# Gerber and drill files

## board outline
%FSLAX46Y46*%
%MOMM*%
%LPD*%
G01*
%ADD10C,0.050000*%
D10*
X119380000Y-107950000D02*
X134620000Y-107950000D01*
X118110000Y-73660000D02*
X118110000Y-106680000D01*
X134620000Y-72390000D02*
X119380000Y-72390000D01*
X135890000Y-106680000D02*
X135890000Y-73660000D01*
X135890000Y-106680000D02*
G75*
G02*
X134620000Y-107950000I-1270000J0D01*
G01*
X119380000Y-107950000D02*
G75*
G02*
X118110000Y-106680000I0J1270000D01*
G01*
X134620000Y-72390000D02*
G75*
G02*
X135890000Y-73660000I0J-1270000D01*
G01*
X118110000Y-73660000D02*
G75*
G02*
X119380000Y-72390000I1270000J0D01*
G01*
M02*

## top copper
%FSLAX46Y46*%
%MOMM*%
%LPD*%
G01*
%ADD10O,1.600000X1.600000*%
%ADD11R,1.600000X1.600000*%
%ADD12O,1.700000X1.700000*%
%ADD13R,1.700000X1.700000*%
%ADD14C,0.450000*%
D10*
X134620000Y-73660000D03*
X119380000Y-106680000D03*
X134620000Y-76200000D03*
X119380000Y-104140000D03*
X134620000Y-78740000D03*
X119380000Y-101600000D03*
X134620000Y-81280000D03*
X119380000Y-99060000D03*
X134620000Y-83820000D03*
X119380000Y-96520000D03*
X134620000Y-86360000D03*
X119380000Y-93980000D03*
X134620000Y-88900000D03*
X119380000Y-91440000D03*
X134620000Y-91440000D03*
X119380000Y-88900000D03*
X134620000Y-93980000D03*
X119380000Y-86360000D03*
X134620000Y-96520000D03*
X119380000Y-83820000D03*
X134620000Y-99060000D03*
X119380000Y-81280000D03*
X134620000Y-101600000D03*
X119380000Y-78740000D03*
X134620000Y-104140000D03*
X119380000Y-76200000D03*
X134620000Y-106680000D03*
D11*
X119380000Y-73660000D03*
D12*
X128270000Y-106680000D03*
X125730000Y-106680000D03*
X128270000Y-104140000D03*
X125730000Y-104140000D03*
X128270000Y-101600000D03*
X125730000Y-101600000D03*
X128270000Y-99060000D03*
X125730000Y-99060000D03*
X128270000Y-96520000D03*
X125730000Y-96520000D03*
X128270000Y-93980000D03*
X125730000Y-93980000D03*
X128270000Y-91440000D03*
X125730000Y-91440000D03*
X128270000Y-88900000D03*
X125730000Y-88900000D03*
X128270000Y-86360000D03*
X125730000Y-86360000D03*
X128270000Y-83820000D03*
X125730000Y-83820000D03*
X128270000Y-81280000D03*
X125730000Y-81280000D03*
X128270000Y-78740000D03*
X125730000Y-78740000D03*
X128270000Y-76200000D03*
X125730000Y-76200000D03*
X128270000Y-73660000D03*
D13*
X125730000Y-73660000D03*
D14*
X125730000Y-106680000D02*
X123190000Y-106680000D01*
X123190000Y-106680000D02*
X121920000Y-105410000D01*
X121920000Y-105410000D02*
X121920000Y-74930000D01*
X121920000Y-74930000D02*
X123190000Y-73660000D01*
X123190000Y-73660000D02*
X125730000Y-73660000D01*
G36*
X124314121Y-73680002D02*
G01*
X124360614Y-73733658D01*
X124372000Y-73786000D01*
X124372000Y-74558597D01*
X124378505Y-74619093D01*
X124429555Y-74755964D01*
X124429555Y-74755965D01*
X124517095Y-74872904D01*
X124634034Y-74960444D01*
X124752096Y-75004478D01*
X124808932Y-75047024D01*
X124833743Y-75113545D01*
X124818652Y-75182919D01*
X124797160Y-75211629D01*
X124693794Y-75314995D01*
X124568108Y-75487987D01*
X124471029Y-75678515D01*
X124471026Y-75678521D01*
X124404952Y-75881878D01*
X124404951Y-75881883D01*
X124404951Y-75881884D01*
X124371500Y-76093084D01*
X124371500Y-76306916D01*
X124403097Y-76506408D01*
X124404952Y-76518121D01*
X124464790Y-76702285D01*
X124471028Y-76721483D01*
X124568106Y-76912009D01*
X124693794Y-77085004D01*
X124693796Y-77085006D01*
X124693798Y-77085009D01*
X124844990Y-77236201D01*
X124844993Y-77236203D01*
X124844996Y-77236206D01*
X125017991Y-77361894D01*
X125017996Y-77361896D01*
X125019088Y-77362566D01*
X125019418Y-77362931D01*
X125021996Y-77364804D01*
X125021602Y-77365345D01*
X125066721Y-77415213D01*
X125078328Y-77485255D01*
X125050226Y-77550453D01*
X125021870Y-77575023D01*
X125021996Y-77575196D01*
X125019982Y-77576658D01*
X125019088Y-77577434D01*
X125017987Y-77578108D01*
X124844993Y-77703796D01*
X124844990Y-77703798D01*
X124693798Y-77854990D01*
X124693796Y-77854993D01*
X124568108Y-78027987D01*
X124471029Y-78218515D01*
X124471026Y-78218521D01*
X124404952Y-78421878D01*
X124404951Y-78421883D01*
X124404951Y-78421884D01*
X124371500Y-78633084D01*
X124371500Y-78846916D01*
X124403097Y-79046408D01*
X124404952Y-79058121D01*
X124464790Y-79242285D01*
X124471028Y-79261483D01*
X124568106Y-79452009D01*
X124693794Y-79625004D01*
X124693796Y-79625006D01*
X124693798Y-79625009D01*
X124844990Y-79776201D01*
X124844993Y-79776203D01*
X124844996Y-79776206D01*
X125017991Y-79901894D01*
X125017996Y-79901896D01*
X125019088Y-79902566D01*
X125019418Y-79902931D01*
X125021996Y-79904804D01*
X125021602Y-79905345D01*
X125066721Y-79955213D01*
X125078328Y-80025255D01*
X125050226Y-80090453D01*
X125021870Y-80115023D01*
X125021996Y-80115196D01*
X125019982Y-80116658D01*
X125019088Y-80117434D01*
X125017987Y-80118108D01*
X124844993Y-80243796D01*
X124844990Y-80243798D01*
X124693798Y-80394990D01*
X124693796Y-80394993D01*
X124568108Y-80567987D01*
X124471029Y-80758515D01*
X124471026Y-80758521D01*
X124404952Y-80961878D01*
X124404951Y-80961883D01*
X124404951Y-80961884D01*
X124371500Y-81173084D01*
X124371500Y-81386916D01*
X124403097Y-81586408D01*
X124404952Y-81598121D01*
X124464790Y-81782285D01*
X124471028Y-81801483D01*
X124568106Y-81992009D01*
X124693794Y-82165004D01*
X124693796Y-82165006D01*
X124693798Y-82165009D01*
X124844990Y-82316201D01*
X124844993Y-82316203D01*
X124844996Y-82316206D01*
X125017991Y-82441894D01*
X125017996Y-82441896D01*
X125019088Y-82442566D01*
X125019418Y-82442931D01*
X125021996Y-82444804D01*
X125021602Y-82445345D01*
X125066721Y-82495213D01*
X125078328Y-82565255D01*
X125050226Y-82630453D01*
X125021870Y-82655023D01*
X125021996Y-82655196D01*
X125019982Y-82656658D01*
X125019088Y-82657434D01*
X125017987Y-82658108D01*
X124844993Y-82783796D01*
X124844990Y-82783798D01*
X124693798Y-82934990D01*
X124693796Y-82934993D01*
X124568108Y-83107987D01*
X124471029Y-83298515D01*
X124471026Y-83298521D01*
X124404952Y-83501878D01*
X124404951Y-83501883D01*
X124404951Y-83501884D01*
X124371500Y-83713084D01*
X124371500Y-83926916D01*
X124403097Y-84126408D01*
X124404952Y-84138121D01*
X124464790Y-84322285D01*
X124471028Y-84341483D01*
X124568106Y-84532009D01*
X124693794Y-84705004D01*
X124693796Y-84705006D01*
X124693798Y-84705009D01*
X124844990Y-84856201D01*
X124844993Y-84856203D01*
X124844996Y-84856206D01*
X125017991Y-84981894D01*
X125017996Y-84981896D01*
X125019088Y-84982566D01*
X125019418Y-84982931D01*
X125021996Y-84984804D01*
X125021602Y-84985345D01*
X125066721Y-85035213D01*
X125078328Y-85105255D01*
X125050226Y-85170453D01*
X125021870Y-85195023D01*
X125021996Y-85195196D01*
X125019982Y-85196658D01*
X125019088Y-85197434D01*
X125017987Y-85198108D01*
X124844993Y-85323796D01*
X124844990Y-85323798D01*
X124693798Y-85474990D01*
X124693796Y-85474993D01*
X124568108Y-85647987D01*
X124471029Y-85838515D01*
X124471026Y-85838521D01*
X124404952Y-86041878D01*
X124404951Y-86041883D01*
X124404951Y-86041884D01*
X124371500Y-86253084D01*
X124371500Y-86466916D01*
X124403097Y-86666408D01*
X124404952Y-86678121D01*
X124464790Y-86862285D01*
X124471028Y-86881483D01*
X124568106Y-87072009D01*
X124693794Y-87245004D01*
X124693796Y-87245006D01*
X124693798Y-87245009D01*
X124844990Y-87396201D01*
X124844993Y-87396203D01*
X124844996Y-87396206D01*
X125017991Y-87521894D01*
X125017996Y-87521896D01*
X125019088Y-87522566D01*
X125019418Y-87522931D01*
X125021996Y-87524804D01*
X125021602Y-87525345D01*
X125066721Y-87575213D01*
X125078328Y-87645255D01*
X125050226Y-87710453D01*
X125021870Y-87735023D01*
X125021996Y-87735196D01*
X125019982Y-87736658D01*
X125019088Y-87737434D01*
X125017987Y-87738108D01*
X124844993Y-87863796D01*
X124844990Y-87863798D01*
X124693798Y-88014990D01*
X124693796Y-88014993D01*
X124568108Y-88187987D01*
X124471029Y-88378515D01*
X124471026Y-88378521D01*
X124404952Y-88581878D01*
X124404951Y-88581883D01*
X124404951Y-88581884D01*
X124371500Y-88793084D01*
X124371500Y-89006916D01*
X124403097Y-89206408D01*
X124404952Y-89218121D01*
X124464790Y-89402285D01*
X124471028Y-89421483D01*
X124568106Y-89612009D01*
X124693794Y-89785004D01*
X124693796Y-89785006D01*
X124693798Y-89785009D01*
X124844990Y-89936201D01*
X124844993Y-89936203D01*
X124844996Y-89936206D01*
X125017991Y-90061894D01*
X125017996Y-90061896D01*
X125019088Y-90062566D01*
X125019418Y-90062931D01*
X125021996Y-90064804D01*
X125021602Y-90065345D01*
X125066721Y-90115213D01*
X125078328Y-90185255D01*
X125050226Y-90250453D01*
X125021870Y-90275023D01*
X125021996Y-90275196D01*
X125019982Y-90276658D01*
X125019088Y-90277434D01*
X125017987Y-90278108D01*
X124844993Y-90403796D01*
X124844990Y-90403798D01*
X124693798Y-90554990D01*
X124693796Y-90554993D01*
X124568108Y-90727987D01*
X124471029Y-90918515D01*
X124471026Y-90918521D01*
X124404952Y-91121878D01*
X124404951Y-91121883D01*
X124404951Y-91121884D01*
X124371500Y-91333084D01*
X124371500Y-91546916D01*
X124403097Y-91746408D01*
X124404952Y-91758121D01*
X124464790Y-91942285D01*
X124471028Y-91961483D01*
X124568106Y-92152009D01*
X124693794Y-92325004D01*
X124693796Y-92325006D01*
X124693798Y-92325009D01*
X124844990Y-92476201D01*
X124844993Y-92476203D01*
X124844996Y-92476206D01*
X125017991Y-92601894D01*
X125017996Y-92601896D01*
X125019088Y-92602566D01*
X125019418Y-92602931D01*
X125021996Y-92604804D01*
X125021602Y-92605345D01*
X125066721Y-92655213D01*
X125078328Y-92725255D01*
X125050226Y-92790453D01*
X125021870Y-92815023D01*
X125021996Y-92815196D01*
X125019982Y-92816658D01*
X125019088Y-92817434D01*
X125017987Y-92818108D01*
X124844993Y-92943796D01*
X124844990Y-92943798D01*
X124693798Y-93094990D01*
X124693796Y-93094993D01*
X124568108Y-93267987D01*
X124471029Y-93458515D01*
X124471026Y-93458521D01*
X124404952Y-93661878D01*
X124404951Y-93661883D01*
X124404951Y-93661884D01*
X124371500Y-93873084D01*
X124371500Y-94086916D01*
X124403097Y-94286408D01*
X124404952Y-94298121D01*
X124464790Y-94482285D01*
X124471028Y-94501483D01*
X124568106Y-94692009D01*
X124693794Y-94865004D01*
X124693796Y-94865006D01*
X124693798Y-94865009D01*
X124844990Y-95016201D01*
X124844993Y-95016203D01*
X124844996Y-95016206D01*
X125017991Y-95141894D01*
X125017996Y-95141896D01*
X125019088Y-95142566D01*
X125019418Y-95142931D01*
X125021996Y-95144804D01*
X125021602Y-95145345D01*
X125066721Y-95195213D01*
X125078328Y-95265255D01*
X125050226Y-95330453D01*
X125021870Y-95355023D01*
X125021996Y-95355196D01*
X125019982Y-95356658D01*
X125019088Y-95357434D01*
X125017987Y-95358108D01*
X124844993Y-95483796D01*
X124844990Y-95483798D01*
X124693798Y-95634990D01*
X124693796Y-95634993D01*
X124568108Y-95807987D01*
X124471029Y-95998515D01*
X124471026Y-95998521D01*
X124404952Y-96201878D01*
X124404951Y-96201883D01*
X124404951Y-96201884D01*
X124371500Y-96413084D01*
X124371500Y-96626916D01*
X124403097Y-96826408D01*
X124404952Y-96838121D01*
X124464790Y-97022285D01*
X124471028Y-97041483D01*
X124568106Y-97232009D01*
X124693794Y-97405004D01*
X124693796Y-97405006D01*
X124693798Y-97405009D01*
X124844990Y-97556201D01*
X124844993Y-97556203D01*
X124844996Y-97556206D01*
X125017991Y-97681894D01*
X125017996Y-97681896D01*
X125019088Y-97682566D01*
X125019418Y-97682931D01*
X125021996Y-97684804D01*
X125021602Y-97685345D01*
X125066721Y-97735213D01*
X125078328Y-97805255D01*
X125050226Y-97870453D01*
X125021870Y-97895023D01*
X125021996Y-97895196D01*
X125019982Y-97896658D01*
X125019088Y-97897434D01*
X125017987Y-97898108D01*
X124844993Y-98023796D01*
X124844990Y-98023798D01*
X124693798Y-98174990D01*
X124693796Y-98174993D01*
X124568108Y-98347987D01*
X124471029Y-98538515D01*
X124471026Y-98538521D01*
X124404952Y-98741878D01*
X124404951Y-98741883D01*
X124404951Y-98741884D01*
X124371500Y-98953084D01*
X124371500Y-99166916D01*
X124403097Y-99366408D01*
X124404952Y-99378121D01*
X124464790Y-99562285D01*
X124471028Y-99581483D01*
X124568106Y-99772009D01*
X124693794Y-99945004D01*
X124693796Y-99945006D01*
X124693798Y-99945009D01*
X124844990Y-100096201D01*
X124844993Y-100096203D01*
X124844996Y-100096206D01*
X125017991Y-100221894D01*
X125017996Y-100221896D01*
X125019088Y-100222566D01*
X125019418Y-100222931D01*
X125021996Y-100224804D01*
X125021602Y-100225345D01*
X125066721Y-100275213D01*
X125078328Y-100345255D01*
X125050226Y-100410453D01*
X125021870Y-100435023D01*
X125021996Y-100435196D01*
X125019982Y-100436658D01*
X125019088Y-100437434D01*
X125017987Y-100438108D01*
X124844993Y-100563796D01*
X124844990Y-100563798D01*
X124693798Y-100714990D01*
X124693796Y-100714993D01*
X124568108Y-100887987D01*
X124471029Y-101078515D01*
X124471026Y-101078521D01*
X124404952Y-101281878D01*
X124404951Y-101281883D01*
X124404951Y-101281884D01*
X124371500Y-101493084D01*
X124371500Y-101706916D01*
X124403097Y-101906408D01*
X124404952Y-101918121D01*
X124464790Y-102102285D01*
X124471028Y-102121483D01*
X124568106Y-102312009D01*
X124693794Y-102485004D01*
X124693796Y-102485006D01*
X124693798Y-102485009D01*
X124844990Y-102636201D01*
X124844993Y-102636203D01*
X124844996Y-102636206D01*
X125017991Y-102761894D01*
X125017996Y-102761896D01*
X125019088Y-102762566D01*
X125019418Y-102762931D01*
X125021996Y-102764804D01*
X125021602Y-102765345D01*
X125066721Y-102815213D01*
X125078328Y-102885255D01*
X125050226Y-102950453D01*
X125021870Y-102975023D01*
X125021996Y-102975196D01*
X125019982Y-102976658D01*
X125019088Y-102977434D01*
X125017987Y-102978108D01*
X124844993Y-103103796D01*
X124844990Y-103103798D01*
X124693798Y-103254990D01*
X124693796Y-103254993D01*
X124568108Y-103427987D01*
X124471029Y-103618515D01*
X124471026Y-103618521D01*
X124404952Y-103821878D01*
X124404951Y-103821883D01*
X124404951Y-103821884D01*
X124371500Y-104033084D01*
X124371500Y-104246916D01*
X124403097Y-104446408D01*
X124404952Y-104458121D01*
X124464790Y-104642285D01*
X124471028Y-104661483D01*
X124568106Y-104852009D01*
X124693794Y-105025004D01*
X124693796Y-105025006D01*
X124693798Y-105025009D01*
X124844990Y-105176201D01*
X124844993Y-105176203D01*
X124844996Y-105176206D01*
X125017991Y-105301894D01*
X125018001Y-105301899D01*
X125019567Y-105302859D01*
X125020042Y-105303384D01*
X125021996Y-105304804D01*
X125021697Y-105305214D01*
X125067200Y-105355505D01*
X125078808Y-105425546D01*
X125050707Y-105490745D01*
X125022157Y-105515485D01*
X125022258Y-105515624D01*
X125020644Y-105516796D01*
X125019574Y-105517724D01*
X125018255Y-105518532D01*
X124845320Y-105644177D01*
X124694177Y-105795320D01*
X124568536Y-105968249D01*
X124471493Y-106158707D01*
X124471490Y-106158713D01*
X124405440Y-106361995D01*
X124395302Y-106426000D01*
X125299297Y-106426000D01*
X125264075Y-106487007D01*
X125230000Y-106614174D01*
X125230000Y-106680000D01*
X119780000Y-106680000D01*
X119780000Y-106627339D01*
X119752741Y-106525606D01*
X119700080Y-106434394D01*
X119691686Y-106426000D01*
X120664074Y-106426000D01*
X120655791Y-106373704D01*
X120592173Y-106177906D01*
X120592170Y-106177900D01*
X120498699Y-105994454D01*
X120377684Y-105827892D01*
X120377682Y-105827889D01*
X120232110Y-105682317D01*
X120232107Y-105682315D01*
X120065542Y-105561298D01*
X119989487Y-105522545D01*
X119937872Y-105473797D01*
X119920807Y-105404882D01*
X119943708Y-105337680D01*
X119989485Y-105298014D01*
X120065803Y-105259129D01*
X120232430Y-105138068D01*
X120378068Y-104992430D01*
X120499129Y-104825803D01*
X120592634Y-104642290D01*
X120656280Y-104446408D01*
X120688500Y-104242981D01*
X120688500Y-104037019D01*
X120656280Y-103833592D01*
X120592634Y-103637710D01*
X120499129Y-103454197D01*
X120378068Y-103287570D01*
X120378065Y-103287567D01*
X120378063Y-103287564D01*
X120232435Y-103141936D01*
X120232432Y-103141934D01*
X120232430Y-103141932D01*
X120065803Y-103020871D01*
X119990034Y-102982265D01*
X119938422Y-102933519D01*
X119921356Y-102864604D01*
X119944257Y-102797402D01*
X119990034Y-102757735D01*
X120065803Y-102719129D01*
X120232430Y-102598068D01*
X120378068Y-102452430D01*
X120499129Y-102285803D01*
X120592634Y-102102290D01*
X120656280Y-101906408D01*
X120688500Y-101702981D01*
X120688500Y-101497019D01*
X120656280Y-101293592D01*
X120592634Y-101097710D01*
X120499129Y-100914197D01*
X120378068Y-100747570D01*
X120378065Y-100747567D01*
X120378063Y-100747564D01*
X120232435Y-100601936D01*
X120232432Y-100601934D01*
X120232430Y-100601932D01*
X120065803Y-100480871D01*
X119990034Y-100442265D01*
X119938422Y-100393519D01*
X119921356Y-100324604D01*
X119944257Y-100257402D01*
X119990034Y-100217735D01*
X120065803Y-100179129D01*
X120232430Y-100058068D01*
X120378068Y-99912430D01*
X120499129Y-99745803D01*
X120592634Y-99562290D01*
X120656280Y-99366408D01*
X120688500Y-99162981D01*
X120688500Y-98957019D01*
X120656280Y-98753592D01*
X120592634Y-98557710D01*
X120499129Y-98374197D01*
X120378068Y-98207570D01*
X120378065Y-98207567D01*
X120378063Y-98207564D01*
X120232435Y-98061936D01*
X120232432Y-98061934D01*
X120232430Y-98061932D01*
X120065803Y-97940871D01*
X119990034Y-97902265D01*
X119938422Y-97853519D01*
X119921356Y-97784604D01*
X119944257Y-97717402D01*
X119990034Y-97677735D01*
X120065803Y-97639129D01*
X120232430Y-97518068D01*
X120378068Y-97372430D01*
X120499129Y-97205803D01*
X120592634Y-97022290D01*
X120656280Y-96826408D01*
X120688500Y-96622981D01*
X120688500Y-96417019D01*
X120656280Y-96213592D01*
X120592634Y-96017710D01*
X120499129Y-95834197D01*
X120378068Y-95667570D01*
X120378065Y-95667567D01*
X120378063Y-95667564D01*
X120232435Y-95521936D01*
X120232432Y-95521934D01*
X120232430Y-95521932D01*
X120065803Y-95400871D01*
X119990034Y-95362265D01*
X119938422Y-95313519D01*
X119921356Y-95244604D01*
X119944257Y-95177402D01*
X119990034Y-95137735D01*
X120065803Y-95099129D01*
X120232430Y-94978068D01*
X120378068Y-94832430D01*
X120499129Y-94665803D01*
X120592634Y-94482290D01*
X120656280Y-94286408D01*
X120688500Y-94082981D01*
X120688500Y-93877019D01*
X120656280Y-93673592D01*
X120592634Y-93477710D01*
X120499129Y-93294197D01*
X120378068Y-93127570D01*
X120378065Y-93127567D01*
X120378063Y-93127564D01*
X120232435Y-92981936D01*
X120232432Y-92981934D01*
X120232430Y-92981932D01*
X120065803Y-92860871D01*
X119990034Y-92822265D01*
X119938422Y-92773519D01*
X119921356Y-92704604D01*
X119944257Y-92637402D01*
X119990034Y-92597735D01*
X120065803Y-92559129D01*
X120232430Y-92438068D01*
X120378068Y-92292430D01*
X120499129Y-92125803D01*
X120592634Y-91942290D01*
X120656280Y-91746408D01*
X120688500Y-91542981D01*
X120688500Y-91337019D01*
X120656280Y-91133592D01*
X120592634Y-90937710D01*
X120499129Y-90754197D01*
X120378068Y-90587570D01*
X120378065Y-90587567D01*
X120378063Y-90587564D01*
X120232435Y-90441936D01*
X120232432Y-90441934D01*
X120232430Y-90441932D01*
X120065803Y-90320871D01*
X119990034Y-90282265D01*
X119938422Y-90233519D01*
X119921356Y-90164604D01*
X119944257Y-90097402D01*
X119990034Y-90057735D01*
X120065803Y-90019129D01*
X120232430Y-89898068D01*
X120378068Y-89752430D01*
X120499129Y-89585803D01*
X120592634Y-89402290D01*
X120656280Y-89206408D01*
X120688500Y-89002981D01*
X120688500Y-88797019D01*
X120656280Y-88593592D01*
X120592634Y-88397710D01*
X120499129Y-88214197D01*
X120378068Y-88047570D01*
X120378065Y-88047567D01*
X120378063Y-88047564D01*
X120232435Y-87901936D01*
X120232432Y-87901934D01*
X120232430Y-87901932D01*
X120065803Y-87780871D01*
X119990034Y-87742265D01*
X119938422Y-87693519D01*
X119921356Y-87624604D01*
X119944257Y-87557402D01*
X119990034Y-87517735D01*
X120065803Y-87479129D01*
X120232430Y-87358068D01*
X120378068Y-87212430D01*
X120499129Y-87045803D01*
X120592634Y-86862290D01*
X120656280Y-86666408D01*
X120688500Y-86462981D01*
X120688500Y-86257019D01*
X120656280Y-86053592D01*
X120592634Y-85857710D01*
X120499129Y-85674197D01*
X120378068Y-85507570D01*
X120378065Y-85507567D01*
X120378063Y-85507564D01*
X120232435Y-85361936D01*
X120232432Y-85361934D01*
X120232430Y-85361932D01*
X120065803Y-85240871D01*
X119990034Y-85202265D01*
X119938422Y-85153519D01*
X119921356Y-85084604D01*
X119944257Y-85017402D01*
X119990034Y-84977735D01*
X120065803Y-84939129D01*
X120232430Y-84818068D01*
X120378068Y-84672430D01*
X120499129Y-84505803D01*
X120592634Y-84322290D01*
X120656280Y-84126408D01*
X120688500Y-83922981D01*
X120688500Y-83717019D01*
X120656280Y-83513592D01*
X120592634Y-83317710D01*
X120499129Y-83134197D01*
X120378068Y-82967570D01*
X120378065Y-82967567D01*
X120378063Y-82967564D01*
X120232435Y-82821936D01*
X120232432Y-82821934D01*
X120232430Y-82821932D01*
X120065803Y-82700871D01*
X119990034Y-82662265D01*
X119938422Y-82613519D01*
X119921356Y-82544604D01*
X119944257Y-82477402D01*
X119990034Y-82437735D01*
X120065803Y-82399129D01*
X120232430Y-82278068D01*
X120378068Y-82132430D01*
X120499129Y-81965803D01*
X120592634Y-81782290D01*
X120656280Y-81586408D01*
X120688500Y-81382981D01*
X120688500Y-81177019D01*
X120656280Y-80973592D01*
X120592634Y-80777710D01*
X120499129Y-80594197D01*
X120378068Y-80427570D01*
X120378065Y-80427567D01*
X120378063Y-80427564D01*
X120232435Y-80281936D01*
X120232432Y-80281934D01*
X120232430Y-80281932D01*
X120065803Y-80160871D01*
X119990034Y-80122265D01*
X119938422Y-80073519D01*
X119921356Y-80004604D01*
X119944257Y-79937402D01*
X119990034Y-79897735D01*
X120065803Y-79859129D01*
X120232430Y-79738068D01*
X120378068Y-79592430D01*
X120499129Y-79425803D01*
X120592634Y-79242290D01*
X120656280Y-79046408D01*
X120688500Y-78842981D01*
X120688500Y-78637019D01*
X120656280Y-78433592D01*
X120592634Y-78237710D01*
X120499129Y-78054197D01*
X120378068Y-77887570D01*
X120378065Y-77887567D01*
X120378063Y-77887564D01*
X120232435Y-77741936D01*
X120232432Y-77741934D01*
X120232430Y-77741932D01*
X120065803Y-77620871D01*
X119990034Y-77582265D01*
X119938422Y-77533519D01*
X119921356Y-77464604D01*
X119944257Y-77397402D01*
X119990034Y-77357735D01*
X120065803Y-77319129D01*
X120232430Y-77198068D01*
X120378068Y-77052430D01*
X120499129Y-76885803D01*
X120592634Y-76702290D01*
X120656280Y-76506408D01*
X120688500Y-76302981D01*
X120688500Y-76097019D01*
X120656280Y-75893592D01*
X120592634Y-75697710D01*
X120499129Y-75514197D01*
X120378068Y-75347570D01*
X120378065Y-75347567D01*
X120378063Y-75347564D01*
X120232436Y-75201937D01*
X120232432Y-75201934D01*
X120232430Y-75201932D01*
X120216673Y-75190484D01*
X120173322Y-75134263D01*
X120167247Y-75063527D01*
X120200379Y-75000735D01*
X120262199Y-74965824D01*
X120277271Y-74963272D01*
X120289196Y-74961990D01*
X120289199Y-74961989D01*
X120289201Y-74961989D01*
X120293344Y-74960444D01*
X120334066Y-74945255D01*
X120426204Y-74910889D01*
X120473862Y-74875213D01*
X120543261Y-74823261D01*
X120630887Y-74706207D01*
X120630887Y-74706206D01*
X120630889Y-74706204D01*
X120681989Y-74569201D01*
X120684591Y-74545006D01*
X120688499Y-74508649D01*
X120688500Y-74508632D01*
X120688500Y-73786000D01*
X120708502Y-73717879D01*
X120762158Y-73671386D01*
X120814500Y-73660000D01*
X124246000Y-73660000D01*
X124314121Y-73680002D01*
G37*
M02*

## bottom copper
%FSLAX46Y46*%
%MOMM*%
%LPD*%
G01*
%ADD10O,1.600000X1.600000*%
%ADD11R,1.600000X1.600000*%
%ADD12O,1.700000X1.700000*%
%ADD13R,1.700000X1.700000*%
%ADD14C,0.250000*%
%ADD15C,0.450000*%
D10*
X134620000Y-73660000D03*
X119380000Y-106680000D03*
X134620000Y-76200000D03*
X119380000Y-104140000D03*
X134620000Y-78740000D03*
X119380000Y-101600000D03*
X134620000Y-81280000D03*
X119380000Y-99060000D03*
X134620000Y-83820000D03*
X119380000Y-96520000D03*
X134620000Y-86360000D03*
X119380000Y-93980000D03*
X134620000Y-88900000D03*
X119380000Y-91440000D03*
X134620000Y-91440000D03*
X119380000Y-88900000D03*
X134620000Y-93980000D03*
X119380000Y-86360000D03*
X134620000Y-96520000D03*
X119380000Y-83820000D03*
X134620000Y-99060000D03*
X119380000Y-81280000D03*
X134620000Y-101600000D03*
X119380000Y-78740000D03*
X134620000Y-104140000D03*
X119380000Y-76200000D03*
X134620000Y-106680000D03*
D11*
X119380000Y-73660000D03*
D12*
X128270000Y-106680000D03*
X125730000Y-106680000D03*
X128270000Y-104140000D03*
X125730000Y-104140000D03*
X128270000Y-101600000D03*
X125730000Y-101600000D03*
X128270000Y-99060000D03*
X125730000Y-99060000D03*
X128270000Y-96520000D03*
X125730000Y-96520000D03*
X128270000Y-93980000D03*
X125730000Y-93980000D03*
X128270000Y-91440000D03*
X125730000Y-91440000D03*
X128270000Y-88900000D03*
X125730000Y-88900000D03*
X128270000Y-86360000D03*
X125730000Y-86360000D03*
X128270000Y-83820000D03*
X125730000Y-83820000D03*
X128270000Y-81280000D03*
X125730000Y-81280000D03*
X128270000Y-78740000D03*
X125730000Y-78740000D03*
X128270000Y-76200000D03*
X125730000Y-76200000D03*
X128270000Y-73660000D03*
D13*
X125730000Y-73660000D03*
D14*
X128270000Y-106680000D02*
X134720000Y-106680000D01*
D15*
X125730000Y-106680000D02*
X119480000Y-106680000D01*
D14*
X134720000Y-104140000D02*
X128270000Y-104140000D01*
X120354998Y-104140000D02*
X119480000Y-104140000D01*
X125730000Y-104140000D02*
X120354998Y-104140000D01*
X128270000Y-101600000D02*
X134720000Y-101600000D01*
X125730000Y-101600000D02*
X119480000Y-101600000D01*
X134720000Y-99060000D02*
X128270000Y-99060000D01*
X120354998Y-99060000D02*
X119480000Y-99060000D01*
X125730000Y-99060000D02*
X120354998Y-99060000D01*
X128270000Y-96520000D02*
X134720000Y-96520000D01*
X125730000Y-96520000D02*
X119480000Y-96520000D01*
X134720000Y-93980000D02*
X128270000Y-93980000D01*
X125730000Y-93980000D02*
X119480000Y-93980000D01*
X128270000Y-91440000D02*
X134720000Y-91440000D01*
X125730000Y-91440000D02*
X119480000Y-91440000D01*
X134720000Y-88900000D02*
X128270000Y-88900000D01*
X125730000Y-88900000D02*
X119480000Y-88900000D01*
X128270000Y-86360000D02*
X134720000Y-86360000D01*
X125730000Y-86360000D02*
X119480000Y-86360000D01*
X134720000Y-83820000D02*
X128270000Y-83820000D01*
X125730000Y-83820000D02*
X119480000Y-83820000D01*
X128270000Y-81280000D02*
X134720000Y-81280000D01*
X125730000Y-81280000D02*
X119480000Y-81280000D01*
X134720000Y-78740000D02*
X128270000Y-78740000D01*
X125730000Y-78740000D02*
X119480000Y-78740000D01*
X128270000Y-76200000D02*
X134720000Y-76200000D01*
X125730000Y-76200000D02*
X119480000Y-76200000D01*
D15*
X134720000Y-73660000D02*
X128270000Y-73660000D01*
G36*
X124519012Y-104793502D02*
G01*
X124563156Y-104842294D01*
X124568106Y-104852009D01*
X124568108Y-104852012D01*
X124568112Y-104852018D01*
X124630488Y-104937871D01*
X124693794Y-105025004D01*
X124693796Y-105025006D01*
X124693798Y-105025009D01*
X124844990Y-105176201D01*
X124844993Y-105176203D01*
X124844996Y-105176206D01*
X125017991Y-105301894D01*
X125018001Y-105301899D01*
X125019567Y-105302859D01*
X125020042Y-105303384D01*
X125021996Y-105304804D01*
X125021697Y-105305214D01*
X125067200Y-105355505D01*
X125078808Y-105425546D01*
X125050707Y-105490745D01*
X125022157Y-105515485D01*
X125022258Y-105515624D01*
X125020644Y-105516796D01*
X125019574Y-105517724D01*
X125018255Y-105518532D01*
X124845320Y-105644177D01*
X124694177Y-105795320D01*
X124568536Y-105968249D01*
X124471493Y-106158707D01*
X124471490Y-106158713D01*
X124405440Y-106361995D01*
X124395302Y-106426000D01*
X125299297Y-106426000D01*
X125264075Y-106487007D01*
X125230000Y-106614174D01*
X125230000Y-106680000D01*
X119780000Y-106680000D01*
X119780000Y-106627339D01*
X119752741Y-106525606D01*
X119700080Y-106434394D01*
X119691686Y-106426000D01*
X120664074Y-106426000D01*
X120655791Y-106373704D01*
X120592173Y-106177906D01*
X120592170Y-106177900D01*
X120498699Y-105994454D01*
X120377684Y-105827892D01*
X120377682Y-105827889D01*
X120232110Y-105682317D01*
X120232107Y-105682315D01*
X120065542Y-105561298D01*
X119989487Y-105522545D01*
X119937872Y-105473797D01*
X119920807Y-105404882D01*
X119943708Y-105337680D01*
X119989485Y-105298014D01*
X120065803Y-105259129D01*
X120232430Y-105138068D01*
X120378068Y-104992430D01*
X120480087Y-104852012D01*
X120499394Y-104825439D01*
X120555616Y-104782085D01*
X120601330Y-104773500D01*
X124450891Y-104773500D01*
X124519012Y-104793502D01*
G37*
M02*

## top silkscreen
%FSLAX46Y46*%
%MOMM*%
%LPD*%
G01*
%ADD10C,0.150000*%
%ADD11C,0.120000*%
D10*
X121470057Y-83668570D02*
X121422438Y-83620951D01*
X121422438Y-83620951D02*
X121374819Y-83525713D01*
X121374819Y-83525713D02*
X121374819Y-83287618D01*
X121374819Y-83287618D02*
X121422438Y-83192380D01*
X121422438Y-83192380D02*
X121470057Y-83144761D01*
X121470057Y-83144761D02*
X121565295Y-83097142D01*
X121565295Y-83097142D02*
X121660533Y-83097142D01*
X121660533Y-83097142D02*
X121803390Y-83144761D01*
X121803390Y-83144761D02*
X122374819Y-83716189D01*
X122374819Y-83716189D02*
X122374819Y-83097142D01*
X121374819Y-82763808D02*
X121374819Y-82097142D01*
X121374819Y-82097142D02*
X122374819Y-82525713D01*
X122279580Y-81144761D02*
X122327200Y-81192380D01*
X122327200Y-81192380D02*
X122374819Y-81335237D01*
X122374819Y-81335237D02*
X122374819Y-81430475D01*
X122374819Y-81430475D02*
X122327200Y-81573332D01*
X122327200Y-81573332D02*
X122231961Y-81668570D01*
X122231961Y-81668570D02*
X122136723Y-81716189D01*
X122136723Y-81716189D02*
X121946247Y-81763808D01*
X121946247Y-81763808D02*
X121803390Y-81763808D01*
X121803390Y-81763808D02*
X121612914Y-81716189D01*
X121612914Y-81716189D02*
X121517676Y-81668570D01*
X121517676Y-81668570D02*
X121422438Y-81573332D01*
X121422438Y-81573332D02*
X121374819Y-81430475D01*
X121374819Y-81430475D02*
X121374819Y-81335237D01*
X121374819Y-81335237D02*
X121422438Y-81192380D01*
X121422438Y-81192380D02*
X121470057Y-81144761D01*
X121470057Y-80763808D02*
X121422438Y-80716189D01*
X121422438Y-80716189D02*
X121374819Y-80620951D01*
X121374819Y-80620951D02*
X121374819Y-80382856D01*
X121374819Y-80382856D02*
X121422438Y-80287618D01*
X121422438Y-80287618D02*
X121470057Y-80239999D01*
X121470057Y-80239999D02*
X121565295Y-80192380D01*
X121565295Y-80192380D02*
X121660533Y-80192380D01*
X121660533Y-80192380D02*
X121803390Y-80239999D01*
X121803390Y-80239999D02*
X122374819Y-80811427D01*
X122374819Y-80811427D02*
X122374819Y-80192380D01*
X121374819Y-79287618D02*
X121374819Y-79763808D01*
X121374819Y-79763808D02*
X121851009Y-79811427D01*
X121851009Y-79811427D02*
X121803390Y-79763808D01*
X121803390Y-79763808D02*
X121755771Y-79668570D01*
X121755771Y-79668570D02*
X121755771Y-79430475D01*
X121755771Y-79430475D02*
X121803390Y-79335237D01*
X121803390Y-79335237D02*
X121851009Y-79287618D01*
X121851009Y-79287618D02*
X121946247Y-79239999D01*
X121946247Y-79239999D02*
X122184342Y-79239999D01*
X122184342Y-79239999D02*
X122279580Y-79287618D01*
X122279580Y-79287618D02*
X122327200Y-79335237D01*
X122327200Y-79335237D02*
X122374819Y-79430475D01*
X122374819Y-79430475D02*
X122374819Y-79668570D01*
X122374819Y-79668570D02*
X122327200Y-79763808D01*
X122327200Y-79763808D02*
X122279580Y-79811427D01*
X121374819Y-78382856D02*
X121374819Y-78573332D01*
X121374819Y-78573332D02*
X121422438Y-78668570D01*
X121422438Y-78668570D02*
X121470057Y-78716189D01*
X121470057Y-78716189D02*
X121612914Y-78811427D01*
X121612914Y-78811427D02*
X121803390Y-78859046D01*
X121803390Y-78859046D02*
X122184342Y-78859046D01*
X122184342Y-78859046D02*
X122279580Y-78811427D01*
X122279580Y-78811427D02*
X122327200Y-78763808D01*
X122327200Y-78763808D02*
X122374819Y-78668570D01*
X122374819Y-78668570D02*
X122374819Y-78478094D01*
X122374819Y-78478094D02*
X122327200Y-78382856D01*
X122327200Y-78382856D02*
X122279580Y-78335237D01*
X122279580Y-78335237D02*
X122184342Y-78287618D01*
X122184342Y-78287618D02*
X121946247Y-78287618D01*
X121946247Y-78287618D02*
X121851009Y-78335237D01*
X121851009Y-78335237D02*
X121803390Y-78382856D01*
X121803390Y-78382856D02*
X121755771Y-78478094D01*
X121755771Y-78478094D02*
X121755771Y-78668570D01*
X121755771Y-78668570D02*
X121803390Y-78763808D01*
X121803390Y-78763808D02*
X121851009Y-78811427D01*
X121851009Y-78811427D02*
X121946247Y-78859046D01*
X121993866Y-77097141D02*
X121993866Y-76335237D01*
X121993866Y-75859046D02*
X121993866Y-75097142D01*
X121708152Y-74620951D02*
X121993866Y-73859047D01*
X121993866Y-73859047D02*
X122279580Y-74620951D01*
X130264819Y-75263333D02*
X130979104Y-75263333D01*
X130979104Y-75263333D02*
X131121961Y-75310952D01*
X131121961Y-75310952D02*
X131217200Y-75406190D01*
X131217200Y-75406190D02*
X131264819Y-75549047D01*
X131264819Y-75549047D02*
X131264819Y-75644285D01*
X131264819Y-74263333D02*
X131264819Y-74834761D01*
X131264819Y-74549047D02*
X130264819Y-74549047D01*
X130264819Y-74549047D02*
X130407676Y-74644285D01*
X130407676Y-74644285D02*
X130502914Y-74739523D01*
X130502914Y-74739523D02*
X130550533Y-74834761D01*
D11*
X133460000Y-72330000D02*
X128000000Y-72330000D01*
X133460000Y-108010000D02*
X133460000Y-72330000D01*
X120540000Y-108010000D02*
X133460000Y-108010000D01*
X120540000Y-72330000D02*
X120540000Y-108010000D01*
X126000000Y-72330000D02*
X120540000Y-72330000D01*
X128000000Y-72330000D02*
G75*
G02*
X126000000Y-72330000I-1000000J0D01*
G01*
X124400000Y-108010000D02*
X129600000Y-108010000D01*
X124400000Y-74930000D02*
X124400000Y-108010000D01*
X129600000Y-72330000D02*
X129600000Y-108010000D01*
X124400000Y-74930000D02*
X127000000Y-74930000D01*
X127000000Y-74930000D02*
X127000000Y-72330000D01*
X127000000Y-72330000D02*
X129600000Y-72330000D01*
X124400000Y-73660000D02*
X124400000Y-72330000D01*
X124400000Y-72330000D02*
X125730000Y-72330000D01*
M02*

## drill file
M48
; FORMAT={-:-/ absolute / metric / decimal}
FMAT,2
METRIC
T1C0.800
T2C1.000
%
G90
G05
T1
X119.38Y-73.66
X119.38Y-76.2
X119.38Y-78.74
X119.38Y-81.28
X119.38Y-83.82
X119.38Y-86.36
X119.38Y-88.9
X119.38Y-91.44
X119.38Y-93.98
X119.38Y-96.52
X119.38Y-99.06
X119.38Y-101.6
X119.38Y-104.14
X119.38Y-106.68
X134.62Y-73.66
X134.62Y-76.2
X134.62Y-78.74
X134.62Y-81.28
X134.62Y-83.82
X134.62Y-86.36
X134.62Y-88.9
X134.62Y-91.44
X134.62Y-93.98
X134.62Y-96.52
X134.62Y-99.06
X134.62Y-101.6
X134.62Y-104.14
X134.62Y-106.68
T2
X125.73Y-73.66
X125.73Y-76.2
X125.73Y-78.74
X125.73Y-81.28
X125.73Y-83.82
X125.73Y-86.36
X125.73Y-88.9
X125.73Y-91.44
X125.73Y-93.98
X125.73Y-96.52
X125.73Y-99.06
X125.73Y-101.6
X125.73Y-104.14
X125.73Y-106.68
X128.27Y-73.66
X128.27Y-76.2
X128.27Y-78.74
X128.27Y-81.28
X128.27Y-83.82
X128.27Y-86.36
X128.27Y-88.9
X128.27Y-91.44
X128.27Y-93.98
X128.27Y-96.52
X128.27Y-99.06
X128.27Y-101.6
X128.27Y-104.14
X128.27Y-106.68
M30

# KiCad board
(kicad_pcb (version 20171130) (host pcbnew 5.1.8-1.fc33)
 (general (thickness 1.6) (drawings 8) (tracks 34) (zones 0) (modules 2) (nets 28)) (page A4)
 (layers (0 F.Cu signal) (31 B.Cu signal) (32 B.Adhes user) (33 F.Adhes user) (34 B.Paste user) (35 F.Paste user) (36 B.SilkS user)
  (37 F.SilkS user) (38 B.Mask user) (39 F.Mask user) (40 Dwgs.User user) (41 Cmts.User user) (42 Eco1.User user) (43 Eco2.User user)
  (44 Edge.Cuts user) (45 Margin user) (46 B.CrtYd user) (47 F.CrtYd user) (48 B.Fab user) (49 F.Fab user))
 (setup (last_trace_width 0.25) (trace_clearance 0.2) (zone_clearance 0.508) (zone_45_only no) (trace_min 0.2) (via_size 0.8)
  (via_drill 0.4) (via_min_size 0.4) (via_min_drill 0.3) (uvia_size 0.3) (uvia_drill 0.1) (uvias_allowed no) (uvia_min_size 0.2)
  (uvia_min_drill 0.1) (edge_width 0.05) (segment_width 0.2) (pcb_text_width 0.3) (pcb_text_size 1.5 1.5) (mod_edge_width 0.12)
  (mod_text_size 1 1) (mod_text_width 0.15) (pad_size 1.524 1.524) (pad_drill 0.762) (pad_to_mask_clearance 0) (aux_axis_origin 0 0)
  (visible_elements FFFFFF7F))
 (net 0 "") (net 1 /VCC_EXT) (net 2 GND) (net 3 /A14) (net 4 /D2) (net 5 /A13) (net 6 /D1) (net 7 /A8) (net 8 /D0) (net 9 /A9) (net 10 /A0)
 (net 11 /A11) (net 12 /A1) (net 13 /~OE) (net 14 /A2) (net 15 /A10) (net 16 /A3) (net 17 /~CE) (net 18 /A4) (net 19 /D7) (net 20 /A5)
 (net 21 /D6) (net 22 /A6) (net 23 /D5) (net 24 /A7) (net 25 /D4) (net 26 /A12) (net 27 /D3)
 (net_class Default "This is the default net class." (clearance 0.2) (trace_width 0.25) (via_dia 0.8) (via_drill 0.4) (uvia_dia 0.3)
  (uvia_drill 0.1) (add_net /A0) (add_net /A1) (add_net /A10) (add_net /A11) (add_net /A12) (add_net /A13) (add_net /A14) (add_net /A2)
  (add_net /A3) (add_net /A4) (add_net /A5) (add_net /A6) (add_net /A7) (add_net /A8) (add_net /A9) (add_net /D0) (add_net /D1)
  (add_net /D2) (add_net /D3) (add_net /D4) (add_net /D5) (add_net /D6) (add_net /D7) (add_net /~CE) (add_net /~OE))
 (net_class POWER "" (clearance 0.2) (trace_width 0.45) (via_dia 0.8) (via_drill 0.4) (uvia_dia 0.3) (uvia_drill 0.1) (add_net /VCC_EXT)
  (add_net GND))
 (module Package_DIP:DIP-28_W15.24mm (layer F.Cu) (at 119.38 73.66)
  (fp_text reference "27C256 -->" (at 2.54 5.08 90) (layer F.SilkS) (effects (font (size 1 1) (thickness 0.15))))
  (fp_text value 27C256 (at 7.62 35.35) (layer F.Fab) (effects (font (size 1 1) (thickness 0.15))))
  (fp_line (start 14.08 -1.33) (end 8.62 -1.33) (layer F.SilkS) (width 0.12))
  (fp_line (start 14.08 34.35) (end 14.08 -1.33) (layer F.SilkS) (width 0.12))
  (fp_line (start 1.16 34.35) (end 14.08 34.35) (layer F.SilkS) (width 0.12))
  (fp_line (start 1.16 -1.33) (end 1.16 34.35) (layer F.SilkS) (width 0.12))
  (fp_line (start 6.62 -1.33) (end 1.16 -1.33) (layer F.SilkS) (width 0.12))
  (fp_arc (start 7.62 -1.33) (end 6.62 -1.33) (angle -180) (layer F.SilkS) (width 0.12))
  (pad 28 thru_hole oval (at 15.24 0) (size 1.6 1.6) (drill 0.8) (layers *.Cu *.Mask) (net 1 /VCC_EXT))
  (pad 14 thru_hole oval (at 0 33.02) (size 1.6 1.6) (drill 0.8) (layers *.Cu *.Mask) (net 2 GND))
  (pad 27 thru_hole oval (at 15.24 2.54) (size 1.6 1.6) (drill 0.8) (layers *.Cu *.Mask) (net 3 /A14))
  (pad 13 thru_hole oval (at 0 30.48) (size 1.6 1.6) (drill 0.8) (layers *.Cu *.Mask) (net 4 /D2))
  (pad 26 thru_hole oval (at 15.24 5.08) (size 1.6 1.6) (drill 0.8) (layers *.Cu *.Mask) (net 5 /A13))
  (pad 12 thru_hole oval (at 0 27.94) (size 1.6 1.6) (drill 0.8) (layers *.Cu *.Mask) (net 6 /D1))
  (pad 25 thru_hole oval (at 15.24 7.62) (size 1.6 1.6) (drill 0.8) (layers *.Cu *.Mask) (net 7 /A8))
  (pad 11 thru_hole oval (at 0 25.4) (size 1.6 1.6) (drill 0.8) (layers *.Cu *.Mask) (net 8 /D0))
  (pad 24 thru_hole oval (at 15.24 10.16) (size 1.6 1.6) (drill 0.8) (layers *.Cu *.Mask) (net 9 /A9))
  (pad 10 thru_hole oval (at 0 22.86) (size 1.6 1.6) (drill 0.8) (layers *.Cu *.Mask) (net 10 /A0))
  (pad 23 thru_hole oval (at 15.24 12.7) (size 1.6 1.6) (drill 0.8) (layers *.Cu *.Mask) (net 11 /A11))
  (pad 9 thru_hole oval (at 0 20.32) (size 1.6 1.6) (drill 0.8) (layers *.Cu *.Mask) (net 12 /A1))
  (pad 22 thru_hole oval (at 15.24 15.24) (size 1.6 1.6) (drill 0.8) (layers *.Cu *.Mask) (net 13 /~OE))
  (pad 8 thru_hole oval (at 0 17.78) (size 1.6 1.6) (drill 0.8) (layers *.Cu *.Mask) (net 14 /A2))
  (pad 21 thru_hole oval (at 15.24 17.78) (size 1.6 1.6) (drill 0.8) (layers *.Cu *.Mask) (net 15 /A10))
  (pad 7 thru_hole oval (at 0 15.24) (size 1.6 1.6) (drill 0.8) (layers *.Cu *.Mask) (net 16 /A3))
  (pad 20 thru_hole oval (at 15.24 20.32) (size 1.6 1.6) (drill 0.8) (layers *.Cu *.Mask) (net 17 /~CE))
  (pad 6 thru_hole oval (at 0 12.7) (size 1.6 1.6) (drill 0.8) (layers *.Cu *.Mask) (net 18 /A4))
  (pad 19 thru_hole oval (at 15.24 22.86) (size 1.6 1.6) (drill 0.8) (layers *.Cu *.Mask) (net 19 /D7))
  (pad 5 thru_hole oval (at 0 10.16) (size 1.6 1.6) (drill 0.8) (layers *.Cu *.Mask) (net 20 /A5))
  (pad 18 thru_hole oval (at 15.24 25.4) (size 1.6 1.6) (drill 0.8) (layers *.Cu *.Mask) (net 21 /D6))
  (pad 4 thru_hole oval (at 0 7.62) (size 1.6 1.6) (drill 0.8) (layers *.Cu *.Mask) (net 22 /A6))
  (pad 17 thru_hole oval (at 15.24 27.94) (size 1.6 1.6) (drill 0.8) (layers *.Cu *.Mask) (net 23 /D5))
  (pad 3 thru_hole oval (at 0 5.08) (size 1.6 1.6) (drill 0.8) (layers *.Cu *.Mask) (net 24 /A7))
  (pad 16 thru_hole oval (at 15.24 30.48) (size 1.6 1.6) (drill 0.8) (layers *.Cu *.Mask) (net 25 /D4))
  (pad 2 thru_hole oval (at 0 2.54) (size 1.6 1.6) (drill 0.8) (layers *.Cu *.Mask) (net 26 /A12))
  (pad 15 thru_hole oval (at 15.24 33.02) (size 1.6 1.6) (drill 0.8) (layers *.Cu *.Mask) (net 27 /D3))
  (pad 1 thru_hole rect (at 0 0) (size 1.6 1.6) (drill 0.8) (layers *.Cu *.Mask)))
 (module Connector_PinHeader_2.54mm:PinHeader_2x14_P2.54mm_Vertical (layer F.Cu) (at 125.73 73.66)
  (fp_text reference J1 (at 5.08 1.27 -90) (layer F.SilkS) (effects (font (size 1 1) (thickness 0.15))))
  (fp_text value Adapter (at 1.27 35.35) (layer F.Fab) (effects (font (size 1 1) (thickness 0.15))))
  (fp_line (start -1.33 34.35) (end 3.87 34.35) (layer F.SilkS) (width 0.12))
  (fp_line (start -1.33 1.27) (end -1.33 34.35) (layer F.SilkS) (width 0.12))
  (fp_line (start 3.87 -1.33) (end 3.87 34.35) (layer F.SilkS) (width 0.12))
  (fp_line (start -1.33 1.27) (end 1.27 1.27) (layer F.SilkS) (width 0.12))
  (fp_line (start 1.27 1.27) (end 1.27 -1.33) (layer F.SilkS) (width 0.12))
  (fp_line (start 1.27 -1.33) (end 3.87 -1.33) (layer F.SilkS) (width 0.12))
  (fp_line (start -1.33 0) (end -1.33 -1.33) (layer F.SilkS) (width 0.12))
  (fp_line (start -1.33 -1.33) (end 0 -1.33) (layer F.SilkS) (width 0.12))
  (pad 28 thru_hole oval (at 2.54 33.02) (size 1.7 1.7) (drill 1) (layers *.Cu *.Mask) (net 27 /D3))
  (pad 27 thru_hole oval (at 0 33.02) (size 1.7 1.7) (drill 1) (layers *.Cu *.Mask) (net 2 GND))
  (pad 26 thru_hole oval (at 2.54 30.48) (size 1.7 1.7) (drill 1) (layers *.Cu *.Mask) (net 25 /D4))
  (pad 25 thru_hole oval (at 0 30.48) (size 1.7 1.7) (drill 1) (layers *.Cu *.Mask) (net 4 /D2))
  (pad 24 thru_hole oval (at 2.54 27.94) (size 1.7 1.7) (drill 1) (layers *.Cu *.Mask) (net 23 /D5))
  (pad 23 thru_hole oval (at 0 27.94) (size 1.7 1.7) (drill 1) (layers *.Cu *.Mask) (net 6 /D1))
  (pad 22 thru_hole oval (at 2.54 25.4) (size 1.7 1.7) (drill 1) (layers *.Cu *.Mask) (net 21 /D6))
  (pad 21 thru_hole oval (at 0 25.4) (size 1.7 1.7) (drill 1) (layers *.Cu *.Mask) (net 8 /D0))
  (pad 20 thru_hole oval (at 2.54 22.86) (size 1.7 1.7) (drill 1) (layers *.Cu *.Mask) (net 19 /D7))
  (pad 19 thru_hole oval (at 0 22.86) (size 1.7 1.7) (drill 1) (layers *.Cu *.Mask) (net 10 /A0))
  (pad 18 thru_hole oval (at 2.54 20.32) (size 1.7 1.7) (drill 1) (layers *.Cu *.Mask) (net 17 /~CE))
  (pad 17 thru_hole oval (at 0 20.32) (size 1.7 1.7) (drill 1) (layers *.Cu *.Mask) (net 12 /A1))
  (pad 16 thru_hole oval (at 2.54 17.78) (size 1.7 1.7) (drill 1) (layers *.Cu *.Mask) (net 15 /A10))
  (pad 15 thru_hole oval (at 0 17.78) (size 1.7 1.7) (drill 1) (layers *.Cu *.Mask) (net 14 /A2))
  (pad 14 thru_hole oval (at 2.54 15.24) (size 1.7 1.7) (drill 1) (layers *.Cu *.Mask) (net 13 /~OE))
  (pad 13 thru_hole oval (at 0 15.24) (size 1.7 1.7) (drill 1) (layers *.Cu *.Mask) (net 16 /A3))
  (pad 12 thru_hole oval (at 2.54 12.7) (size 1.7 1.7) (drill 1) (layers *.Cu *.Mask) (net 11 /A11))
  (pad 11 thru_hole oval (at 0 12.7) (size 1.7 1.7) (drill 1) (layers *.Cu *.Mask) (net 18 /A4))
  (pad 10 thru_hole oval (at 2.54 10.16) (size 1.7 1.7) (drill 1) (layers *.Cu *.Mask) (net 9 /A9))
  (pad 9 thru_hole oval (at 0 10.16) (size 1.7 1.7) (drill 1) (layers *.Cu *.Mask) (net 20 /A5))
  (pad 8 thru_hole oval (at 2.54 7.62) (size 1.7 1.7) (drill 1) (layers *.Cu *.Mask) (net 7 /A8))
  (pad 7 thru_hole oval (at 0 7.62) (size 1.7 1.7) (drill 1) (layers *.Cu *.Mask) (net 22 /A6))
  (pad 6 thru_hole oval (at 2.54 5.08) (size 1.7 1.7) (drill 1) (layers *.Cu *.Mask) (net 5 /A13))
  (pad 5 thru_hole oval (at 0 5.08) (size 1.7 1.7) (drill 1) (layers *.Cu *.Mask) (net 24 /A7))
  (pad 4 thru_hole oval (at 2.54 2.54) (size 1.7 1.7) (drill 1) (layers *.Cu *.Mask) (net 3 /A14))
  (pad 3 thru_hole oval (at 0 2.54) (size 1.7 1.7) (drill 1) (layers *.Cu *.Mask) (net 26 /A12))
  (pad 2 thru_hole oval (at 2.54 0) (size 1.7 1.7) (drill 1) (layers *.Cu *.Mask) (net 1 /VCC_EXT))
  (pad 1 thru_hole rect (at 0 0) (size 1.7 1.7) (drill 1) (layers *.Cu *.Mask) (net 2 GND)))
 (gr_line (start 119.38 107.95) (end 134.62 107.95) (layer Edge.Cuts) (width 0.05))
 (gr_line (start 118.11 73.66) (end 118.11 106.68) (layer Edge.Cuts) (width 0.05))
 (gr_line (start 134.62 72.39) (end 119.38 72.39) (layer Edge.Cuts) (width 0.05))
 (gr_line (start 135.89 106.68) (end 135.89 73.66) (layer Edge.Cuts) (width 0.05))
 (gr_arc (start 134.62 106.68) (end 134.62 107.95) (angle -90) (layer Edge.Cuts) (width 0.05))
 (gr_arc (start 119.38 106.68) (end 118.11 106.68) (angle -90) (layer Edge.Cuts) (width 0.05))
 (gr_arc (start 134.62 73.66) (end 135.89 73.66) (angle -90) (layer Edge.Cuts) (width 0.05))
 (gr_arc (start 119.38 73.66) (end 119.38 72.39) (angle -90) (layer Edge.Cuts) (width 0.05))
 (segment (start 128.27 106.68) (end 134.72 106.68) (width 0.25) (layer B.Cu) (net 27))
 (segment (start 125.73 106.68) (end 119.48 106.68) (width 0.45) (layer B.Cu) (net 2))
 (segment (start 125.73 106.68) (end 123.19 106.68) (width 0.45) (layer F.Cu) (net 2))
 (segment (start 123.19 106.68) (end 121.92 105.41) (width 0.45) (layer F.Cu) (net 2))
 (segment (start 121.92 105.41) (end 121.92 74.93) (width 0.45) (layer F.Cu) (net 2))
 (segment (start 121.92 74.93) (end 123.19 73.66) (width 0.45) (layer F.Cu) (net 2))
 (segment (start 123.19 73.66) (end 125.73 73.66) (width 0.45) (layer F.Cu) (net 2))
 (segment (start 134.72 104.14) (end 128.27 104.14) (width 0.25) (layer B.Cu) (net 25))
 (segment (start 120.354998 104.14) (end 119.48 104.14) (width 0.25) (layer B.Cu) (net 4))
 (segment (start 125.73 104.14) (end 120.354998 104.14) (width 0.25) (layer B.Cu) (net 4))
 (segment (start 128.27 101.6) (end 134.72 101.6) (width 0.25) (layer B.Cu) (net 23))
 (segment (start 125.73 101.6) (end 119.48 101.6) (width 0.25) (layer B.Cu) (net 6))
 (segment (start 134.72 99.06) (end 128.27 99.06) (width 0.25) (layer B.Cu) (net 21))
 (segment (start 120.354998 99.06) (end 119.48 99.06) (width 0.25) (layer B.Cu) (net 8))
 (segment (start 125.73 99.06) (end 120.354998 99.06) (width 0.25) (layer B.Cu) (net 8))
 (segment (start 128.27 96.52) (end 134.72 96.52) (width 0.25) (layer B.Cu) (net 19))
 (segment (start 125.73 96.52) (end 119.48 96.52) (width 0.25) (layer B.Cu) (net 10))
 (segment (start 134.72 93.98) (end 128.27 93.98) (width 0.25) (layer B.Cu) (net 17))
 (segment (start 125.73 93.98) (end 119.48 93.98) (width 0.25) (layer B.Cu) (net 12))
 (segment (start 128.27 91.44) (end 134.72 91.44) (width 0.25) (layer B.Cu) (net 15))
 (segment (start 125.73 91.44) (end 119.48 91.44) (width 0.25) (layer B.Cu) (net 14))
 (segment (start 134.72 88.9) (end 128.27 88.9) (width 0.25) (layer B.Cu) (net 13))
 (segment (start 125.73 88.9) (end 119.48 88.9) (width 0.25) (layer B.Cu) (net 16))
 (segment (start 128.27 86.36) (end 134.72 86.36) (width 0.25) (layer B.Cu) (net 11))
 (segment (start 125.73 86.36) (end 119.48 86.36) (width 0.25) (layer B.Cu) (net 18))
 (segment (start 134.72 83.82) (end 128.27 83.82) (width 0.25) (layer B.Cu) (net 9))
 (segment (start 125.73 83.82) (end 119.48 83.82) (width 0.25) (layer B.Cu) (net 20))
 (segment (start 128.27 81.28) (end 134.72 81.28) (width 0.25) (layer B.Cu) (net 7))
 (segment (start 125.73 81.28) (end 119.48 81.28) (width 0.25) (layer B.Cu) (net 22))
 (segment (start 134.72 78.74) (end 128.27 78.74) (width 0.25) (layer B.Cu) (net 5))
 (segment (start 125.73 78.74) (end 119.48 78.74) (width 0.25) (layer B.Cu) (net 24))
 (segment (start 128.27 76.2) (end 134.72 76.2) (width 0.25) (layer B.Cu) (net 3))
 (segment (start 125.73 76.2) (end 119.48 76.2) (width 0.25) (layer B.Cu) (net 26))
 (segment (start 134.72 73.66) (end 128.27 73.66) (width 0.45) (layer B.Cu) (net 1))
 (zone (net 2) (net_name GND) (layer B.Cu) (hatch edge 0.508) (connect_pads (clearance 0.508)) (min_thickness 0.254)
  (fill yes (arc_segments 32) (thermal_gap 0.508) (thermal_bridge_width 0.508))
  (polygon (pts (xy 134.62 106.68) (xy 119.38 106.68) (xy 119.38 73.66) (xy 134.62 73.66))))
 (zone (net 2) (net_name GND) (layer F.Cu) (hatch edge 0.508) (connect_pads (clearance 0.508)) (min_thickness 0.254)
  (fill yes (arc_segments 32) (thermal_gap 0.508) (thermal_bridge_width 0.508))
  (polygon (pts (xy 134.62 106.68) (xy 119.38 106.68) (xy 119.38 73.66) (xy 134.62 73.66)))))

